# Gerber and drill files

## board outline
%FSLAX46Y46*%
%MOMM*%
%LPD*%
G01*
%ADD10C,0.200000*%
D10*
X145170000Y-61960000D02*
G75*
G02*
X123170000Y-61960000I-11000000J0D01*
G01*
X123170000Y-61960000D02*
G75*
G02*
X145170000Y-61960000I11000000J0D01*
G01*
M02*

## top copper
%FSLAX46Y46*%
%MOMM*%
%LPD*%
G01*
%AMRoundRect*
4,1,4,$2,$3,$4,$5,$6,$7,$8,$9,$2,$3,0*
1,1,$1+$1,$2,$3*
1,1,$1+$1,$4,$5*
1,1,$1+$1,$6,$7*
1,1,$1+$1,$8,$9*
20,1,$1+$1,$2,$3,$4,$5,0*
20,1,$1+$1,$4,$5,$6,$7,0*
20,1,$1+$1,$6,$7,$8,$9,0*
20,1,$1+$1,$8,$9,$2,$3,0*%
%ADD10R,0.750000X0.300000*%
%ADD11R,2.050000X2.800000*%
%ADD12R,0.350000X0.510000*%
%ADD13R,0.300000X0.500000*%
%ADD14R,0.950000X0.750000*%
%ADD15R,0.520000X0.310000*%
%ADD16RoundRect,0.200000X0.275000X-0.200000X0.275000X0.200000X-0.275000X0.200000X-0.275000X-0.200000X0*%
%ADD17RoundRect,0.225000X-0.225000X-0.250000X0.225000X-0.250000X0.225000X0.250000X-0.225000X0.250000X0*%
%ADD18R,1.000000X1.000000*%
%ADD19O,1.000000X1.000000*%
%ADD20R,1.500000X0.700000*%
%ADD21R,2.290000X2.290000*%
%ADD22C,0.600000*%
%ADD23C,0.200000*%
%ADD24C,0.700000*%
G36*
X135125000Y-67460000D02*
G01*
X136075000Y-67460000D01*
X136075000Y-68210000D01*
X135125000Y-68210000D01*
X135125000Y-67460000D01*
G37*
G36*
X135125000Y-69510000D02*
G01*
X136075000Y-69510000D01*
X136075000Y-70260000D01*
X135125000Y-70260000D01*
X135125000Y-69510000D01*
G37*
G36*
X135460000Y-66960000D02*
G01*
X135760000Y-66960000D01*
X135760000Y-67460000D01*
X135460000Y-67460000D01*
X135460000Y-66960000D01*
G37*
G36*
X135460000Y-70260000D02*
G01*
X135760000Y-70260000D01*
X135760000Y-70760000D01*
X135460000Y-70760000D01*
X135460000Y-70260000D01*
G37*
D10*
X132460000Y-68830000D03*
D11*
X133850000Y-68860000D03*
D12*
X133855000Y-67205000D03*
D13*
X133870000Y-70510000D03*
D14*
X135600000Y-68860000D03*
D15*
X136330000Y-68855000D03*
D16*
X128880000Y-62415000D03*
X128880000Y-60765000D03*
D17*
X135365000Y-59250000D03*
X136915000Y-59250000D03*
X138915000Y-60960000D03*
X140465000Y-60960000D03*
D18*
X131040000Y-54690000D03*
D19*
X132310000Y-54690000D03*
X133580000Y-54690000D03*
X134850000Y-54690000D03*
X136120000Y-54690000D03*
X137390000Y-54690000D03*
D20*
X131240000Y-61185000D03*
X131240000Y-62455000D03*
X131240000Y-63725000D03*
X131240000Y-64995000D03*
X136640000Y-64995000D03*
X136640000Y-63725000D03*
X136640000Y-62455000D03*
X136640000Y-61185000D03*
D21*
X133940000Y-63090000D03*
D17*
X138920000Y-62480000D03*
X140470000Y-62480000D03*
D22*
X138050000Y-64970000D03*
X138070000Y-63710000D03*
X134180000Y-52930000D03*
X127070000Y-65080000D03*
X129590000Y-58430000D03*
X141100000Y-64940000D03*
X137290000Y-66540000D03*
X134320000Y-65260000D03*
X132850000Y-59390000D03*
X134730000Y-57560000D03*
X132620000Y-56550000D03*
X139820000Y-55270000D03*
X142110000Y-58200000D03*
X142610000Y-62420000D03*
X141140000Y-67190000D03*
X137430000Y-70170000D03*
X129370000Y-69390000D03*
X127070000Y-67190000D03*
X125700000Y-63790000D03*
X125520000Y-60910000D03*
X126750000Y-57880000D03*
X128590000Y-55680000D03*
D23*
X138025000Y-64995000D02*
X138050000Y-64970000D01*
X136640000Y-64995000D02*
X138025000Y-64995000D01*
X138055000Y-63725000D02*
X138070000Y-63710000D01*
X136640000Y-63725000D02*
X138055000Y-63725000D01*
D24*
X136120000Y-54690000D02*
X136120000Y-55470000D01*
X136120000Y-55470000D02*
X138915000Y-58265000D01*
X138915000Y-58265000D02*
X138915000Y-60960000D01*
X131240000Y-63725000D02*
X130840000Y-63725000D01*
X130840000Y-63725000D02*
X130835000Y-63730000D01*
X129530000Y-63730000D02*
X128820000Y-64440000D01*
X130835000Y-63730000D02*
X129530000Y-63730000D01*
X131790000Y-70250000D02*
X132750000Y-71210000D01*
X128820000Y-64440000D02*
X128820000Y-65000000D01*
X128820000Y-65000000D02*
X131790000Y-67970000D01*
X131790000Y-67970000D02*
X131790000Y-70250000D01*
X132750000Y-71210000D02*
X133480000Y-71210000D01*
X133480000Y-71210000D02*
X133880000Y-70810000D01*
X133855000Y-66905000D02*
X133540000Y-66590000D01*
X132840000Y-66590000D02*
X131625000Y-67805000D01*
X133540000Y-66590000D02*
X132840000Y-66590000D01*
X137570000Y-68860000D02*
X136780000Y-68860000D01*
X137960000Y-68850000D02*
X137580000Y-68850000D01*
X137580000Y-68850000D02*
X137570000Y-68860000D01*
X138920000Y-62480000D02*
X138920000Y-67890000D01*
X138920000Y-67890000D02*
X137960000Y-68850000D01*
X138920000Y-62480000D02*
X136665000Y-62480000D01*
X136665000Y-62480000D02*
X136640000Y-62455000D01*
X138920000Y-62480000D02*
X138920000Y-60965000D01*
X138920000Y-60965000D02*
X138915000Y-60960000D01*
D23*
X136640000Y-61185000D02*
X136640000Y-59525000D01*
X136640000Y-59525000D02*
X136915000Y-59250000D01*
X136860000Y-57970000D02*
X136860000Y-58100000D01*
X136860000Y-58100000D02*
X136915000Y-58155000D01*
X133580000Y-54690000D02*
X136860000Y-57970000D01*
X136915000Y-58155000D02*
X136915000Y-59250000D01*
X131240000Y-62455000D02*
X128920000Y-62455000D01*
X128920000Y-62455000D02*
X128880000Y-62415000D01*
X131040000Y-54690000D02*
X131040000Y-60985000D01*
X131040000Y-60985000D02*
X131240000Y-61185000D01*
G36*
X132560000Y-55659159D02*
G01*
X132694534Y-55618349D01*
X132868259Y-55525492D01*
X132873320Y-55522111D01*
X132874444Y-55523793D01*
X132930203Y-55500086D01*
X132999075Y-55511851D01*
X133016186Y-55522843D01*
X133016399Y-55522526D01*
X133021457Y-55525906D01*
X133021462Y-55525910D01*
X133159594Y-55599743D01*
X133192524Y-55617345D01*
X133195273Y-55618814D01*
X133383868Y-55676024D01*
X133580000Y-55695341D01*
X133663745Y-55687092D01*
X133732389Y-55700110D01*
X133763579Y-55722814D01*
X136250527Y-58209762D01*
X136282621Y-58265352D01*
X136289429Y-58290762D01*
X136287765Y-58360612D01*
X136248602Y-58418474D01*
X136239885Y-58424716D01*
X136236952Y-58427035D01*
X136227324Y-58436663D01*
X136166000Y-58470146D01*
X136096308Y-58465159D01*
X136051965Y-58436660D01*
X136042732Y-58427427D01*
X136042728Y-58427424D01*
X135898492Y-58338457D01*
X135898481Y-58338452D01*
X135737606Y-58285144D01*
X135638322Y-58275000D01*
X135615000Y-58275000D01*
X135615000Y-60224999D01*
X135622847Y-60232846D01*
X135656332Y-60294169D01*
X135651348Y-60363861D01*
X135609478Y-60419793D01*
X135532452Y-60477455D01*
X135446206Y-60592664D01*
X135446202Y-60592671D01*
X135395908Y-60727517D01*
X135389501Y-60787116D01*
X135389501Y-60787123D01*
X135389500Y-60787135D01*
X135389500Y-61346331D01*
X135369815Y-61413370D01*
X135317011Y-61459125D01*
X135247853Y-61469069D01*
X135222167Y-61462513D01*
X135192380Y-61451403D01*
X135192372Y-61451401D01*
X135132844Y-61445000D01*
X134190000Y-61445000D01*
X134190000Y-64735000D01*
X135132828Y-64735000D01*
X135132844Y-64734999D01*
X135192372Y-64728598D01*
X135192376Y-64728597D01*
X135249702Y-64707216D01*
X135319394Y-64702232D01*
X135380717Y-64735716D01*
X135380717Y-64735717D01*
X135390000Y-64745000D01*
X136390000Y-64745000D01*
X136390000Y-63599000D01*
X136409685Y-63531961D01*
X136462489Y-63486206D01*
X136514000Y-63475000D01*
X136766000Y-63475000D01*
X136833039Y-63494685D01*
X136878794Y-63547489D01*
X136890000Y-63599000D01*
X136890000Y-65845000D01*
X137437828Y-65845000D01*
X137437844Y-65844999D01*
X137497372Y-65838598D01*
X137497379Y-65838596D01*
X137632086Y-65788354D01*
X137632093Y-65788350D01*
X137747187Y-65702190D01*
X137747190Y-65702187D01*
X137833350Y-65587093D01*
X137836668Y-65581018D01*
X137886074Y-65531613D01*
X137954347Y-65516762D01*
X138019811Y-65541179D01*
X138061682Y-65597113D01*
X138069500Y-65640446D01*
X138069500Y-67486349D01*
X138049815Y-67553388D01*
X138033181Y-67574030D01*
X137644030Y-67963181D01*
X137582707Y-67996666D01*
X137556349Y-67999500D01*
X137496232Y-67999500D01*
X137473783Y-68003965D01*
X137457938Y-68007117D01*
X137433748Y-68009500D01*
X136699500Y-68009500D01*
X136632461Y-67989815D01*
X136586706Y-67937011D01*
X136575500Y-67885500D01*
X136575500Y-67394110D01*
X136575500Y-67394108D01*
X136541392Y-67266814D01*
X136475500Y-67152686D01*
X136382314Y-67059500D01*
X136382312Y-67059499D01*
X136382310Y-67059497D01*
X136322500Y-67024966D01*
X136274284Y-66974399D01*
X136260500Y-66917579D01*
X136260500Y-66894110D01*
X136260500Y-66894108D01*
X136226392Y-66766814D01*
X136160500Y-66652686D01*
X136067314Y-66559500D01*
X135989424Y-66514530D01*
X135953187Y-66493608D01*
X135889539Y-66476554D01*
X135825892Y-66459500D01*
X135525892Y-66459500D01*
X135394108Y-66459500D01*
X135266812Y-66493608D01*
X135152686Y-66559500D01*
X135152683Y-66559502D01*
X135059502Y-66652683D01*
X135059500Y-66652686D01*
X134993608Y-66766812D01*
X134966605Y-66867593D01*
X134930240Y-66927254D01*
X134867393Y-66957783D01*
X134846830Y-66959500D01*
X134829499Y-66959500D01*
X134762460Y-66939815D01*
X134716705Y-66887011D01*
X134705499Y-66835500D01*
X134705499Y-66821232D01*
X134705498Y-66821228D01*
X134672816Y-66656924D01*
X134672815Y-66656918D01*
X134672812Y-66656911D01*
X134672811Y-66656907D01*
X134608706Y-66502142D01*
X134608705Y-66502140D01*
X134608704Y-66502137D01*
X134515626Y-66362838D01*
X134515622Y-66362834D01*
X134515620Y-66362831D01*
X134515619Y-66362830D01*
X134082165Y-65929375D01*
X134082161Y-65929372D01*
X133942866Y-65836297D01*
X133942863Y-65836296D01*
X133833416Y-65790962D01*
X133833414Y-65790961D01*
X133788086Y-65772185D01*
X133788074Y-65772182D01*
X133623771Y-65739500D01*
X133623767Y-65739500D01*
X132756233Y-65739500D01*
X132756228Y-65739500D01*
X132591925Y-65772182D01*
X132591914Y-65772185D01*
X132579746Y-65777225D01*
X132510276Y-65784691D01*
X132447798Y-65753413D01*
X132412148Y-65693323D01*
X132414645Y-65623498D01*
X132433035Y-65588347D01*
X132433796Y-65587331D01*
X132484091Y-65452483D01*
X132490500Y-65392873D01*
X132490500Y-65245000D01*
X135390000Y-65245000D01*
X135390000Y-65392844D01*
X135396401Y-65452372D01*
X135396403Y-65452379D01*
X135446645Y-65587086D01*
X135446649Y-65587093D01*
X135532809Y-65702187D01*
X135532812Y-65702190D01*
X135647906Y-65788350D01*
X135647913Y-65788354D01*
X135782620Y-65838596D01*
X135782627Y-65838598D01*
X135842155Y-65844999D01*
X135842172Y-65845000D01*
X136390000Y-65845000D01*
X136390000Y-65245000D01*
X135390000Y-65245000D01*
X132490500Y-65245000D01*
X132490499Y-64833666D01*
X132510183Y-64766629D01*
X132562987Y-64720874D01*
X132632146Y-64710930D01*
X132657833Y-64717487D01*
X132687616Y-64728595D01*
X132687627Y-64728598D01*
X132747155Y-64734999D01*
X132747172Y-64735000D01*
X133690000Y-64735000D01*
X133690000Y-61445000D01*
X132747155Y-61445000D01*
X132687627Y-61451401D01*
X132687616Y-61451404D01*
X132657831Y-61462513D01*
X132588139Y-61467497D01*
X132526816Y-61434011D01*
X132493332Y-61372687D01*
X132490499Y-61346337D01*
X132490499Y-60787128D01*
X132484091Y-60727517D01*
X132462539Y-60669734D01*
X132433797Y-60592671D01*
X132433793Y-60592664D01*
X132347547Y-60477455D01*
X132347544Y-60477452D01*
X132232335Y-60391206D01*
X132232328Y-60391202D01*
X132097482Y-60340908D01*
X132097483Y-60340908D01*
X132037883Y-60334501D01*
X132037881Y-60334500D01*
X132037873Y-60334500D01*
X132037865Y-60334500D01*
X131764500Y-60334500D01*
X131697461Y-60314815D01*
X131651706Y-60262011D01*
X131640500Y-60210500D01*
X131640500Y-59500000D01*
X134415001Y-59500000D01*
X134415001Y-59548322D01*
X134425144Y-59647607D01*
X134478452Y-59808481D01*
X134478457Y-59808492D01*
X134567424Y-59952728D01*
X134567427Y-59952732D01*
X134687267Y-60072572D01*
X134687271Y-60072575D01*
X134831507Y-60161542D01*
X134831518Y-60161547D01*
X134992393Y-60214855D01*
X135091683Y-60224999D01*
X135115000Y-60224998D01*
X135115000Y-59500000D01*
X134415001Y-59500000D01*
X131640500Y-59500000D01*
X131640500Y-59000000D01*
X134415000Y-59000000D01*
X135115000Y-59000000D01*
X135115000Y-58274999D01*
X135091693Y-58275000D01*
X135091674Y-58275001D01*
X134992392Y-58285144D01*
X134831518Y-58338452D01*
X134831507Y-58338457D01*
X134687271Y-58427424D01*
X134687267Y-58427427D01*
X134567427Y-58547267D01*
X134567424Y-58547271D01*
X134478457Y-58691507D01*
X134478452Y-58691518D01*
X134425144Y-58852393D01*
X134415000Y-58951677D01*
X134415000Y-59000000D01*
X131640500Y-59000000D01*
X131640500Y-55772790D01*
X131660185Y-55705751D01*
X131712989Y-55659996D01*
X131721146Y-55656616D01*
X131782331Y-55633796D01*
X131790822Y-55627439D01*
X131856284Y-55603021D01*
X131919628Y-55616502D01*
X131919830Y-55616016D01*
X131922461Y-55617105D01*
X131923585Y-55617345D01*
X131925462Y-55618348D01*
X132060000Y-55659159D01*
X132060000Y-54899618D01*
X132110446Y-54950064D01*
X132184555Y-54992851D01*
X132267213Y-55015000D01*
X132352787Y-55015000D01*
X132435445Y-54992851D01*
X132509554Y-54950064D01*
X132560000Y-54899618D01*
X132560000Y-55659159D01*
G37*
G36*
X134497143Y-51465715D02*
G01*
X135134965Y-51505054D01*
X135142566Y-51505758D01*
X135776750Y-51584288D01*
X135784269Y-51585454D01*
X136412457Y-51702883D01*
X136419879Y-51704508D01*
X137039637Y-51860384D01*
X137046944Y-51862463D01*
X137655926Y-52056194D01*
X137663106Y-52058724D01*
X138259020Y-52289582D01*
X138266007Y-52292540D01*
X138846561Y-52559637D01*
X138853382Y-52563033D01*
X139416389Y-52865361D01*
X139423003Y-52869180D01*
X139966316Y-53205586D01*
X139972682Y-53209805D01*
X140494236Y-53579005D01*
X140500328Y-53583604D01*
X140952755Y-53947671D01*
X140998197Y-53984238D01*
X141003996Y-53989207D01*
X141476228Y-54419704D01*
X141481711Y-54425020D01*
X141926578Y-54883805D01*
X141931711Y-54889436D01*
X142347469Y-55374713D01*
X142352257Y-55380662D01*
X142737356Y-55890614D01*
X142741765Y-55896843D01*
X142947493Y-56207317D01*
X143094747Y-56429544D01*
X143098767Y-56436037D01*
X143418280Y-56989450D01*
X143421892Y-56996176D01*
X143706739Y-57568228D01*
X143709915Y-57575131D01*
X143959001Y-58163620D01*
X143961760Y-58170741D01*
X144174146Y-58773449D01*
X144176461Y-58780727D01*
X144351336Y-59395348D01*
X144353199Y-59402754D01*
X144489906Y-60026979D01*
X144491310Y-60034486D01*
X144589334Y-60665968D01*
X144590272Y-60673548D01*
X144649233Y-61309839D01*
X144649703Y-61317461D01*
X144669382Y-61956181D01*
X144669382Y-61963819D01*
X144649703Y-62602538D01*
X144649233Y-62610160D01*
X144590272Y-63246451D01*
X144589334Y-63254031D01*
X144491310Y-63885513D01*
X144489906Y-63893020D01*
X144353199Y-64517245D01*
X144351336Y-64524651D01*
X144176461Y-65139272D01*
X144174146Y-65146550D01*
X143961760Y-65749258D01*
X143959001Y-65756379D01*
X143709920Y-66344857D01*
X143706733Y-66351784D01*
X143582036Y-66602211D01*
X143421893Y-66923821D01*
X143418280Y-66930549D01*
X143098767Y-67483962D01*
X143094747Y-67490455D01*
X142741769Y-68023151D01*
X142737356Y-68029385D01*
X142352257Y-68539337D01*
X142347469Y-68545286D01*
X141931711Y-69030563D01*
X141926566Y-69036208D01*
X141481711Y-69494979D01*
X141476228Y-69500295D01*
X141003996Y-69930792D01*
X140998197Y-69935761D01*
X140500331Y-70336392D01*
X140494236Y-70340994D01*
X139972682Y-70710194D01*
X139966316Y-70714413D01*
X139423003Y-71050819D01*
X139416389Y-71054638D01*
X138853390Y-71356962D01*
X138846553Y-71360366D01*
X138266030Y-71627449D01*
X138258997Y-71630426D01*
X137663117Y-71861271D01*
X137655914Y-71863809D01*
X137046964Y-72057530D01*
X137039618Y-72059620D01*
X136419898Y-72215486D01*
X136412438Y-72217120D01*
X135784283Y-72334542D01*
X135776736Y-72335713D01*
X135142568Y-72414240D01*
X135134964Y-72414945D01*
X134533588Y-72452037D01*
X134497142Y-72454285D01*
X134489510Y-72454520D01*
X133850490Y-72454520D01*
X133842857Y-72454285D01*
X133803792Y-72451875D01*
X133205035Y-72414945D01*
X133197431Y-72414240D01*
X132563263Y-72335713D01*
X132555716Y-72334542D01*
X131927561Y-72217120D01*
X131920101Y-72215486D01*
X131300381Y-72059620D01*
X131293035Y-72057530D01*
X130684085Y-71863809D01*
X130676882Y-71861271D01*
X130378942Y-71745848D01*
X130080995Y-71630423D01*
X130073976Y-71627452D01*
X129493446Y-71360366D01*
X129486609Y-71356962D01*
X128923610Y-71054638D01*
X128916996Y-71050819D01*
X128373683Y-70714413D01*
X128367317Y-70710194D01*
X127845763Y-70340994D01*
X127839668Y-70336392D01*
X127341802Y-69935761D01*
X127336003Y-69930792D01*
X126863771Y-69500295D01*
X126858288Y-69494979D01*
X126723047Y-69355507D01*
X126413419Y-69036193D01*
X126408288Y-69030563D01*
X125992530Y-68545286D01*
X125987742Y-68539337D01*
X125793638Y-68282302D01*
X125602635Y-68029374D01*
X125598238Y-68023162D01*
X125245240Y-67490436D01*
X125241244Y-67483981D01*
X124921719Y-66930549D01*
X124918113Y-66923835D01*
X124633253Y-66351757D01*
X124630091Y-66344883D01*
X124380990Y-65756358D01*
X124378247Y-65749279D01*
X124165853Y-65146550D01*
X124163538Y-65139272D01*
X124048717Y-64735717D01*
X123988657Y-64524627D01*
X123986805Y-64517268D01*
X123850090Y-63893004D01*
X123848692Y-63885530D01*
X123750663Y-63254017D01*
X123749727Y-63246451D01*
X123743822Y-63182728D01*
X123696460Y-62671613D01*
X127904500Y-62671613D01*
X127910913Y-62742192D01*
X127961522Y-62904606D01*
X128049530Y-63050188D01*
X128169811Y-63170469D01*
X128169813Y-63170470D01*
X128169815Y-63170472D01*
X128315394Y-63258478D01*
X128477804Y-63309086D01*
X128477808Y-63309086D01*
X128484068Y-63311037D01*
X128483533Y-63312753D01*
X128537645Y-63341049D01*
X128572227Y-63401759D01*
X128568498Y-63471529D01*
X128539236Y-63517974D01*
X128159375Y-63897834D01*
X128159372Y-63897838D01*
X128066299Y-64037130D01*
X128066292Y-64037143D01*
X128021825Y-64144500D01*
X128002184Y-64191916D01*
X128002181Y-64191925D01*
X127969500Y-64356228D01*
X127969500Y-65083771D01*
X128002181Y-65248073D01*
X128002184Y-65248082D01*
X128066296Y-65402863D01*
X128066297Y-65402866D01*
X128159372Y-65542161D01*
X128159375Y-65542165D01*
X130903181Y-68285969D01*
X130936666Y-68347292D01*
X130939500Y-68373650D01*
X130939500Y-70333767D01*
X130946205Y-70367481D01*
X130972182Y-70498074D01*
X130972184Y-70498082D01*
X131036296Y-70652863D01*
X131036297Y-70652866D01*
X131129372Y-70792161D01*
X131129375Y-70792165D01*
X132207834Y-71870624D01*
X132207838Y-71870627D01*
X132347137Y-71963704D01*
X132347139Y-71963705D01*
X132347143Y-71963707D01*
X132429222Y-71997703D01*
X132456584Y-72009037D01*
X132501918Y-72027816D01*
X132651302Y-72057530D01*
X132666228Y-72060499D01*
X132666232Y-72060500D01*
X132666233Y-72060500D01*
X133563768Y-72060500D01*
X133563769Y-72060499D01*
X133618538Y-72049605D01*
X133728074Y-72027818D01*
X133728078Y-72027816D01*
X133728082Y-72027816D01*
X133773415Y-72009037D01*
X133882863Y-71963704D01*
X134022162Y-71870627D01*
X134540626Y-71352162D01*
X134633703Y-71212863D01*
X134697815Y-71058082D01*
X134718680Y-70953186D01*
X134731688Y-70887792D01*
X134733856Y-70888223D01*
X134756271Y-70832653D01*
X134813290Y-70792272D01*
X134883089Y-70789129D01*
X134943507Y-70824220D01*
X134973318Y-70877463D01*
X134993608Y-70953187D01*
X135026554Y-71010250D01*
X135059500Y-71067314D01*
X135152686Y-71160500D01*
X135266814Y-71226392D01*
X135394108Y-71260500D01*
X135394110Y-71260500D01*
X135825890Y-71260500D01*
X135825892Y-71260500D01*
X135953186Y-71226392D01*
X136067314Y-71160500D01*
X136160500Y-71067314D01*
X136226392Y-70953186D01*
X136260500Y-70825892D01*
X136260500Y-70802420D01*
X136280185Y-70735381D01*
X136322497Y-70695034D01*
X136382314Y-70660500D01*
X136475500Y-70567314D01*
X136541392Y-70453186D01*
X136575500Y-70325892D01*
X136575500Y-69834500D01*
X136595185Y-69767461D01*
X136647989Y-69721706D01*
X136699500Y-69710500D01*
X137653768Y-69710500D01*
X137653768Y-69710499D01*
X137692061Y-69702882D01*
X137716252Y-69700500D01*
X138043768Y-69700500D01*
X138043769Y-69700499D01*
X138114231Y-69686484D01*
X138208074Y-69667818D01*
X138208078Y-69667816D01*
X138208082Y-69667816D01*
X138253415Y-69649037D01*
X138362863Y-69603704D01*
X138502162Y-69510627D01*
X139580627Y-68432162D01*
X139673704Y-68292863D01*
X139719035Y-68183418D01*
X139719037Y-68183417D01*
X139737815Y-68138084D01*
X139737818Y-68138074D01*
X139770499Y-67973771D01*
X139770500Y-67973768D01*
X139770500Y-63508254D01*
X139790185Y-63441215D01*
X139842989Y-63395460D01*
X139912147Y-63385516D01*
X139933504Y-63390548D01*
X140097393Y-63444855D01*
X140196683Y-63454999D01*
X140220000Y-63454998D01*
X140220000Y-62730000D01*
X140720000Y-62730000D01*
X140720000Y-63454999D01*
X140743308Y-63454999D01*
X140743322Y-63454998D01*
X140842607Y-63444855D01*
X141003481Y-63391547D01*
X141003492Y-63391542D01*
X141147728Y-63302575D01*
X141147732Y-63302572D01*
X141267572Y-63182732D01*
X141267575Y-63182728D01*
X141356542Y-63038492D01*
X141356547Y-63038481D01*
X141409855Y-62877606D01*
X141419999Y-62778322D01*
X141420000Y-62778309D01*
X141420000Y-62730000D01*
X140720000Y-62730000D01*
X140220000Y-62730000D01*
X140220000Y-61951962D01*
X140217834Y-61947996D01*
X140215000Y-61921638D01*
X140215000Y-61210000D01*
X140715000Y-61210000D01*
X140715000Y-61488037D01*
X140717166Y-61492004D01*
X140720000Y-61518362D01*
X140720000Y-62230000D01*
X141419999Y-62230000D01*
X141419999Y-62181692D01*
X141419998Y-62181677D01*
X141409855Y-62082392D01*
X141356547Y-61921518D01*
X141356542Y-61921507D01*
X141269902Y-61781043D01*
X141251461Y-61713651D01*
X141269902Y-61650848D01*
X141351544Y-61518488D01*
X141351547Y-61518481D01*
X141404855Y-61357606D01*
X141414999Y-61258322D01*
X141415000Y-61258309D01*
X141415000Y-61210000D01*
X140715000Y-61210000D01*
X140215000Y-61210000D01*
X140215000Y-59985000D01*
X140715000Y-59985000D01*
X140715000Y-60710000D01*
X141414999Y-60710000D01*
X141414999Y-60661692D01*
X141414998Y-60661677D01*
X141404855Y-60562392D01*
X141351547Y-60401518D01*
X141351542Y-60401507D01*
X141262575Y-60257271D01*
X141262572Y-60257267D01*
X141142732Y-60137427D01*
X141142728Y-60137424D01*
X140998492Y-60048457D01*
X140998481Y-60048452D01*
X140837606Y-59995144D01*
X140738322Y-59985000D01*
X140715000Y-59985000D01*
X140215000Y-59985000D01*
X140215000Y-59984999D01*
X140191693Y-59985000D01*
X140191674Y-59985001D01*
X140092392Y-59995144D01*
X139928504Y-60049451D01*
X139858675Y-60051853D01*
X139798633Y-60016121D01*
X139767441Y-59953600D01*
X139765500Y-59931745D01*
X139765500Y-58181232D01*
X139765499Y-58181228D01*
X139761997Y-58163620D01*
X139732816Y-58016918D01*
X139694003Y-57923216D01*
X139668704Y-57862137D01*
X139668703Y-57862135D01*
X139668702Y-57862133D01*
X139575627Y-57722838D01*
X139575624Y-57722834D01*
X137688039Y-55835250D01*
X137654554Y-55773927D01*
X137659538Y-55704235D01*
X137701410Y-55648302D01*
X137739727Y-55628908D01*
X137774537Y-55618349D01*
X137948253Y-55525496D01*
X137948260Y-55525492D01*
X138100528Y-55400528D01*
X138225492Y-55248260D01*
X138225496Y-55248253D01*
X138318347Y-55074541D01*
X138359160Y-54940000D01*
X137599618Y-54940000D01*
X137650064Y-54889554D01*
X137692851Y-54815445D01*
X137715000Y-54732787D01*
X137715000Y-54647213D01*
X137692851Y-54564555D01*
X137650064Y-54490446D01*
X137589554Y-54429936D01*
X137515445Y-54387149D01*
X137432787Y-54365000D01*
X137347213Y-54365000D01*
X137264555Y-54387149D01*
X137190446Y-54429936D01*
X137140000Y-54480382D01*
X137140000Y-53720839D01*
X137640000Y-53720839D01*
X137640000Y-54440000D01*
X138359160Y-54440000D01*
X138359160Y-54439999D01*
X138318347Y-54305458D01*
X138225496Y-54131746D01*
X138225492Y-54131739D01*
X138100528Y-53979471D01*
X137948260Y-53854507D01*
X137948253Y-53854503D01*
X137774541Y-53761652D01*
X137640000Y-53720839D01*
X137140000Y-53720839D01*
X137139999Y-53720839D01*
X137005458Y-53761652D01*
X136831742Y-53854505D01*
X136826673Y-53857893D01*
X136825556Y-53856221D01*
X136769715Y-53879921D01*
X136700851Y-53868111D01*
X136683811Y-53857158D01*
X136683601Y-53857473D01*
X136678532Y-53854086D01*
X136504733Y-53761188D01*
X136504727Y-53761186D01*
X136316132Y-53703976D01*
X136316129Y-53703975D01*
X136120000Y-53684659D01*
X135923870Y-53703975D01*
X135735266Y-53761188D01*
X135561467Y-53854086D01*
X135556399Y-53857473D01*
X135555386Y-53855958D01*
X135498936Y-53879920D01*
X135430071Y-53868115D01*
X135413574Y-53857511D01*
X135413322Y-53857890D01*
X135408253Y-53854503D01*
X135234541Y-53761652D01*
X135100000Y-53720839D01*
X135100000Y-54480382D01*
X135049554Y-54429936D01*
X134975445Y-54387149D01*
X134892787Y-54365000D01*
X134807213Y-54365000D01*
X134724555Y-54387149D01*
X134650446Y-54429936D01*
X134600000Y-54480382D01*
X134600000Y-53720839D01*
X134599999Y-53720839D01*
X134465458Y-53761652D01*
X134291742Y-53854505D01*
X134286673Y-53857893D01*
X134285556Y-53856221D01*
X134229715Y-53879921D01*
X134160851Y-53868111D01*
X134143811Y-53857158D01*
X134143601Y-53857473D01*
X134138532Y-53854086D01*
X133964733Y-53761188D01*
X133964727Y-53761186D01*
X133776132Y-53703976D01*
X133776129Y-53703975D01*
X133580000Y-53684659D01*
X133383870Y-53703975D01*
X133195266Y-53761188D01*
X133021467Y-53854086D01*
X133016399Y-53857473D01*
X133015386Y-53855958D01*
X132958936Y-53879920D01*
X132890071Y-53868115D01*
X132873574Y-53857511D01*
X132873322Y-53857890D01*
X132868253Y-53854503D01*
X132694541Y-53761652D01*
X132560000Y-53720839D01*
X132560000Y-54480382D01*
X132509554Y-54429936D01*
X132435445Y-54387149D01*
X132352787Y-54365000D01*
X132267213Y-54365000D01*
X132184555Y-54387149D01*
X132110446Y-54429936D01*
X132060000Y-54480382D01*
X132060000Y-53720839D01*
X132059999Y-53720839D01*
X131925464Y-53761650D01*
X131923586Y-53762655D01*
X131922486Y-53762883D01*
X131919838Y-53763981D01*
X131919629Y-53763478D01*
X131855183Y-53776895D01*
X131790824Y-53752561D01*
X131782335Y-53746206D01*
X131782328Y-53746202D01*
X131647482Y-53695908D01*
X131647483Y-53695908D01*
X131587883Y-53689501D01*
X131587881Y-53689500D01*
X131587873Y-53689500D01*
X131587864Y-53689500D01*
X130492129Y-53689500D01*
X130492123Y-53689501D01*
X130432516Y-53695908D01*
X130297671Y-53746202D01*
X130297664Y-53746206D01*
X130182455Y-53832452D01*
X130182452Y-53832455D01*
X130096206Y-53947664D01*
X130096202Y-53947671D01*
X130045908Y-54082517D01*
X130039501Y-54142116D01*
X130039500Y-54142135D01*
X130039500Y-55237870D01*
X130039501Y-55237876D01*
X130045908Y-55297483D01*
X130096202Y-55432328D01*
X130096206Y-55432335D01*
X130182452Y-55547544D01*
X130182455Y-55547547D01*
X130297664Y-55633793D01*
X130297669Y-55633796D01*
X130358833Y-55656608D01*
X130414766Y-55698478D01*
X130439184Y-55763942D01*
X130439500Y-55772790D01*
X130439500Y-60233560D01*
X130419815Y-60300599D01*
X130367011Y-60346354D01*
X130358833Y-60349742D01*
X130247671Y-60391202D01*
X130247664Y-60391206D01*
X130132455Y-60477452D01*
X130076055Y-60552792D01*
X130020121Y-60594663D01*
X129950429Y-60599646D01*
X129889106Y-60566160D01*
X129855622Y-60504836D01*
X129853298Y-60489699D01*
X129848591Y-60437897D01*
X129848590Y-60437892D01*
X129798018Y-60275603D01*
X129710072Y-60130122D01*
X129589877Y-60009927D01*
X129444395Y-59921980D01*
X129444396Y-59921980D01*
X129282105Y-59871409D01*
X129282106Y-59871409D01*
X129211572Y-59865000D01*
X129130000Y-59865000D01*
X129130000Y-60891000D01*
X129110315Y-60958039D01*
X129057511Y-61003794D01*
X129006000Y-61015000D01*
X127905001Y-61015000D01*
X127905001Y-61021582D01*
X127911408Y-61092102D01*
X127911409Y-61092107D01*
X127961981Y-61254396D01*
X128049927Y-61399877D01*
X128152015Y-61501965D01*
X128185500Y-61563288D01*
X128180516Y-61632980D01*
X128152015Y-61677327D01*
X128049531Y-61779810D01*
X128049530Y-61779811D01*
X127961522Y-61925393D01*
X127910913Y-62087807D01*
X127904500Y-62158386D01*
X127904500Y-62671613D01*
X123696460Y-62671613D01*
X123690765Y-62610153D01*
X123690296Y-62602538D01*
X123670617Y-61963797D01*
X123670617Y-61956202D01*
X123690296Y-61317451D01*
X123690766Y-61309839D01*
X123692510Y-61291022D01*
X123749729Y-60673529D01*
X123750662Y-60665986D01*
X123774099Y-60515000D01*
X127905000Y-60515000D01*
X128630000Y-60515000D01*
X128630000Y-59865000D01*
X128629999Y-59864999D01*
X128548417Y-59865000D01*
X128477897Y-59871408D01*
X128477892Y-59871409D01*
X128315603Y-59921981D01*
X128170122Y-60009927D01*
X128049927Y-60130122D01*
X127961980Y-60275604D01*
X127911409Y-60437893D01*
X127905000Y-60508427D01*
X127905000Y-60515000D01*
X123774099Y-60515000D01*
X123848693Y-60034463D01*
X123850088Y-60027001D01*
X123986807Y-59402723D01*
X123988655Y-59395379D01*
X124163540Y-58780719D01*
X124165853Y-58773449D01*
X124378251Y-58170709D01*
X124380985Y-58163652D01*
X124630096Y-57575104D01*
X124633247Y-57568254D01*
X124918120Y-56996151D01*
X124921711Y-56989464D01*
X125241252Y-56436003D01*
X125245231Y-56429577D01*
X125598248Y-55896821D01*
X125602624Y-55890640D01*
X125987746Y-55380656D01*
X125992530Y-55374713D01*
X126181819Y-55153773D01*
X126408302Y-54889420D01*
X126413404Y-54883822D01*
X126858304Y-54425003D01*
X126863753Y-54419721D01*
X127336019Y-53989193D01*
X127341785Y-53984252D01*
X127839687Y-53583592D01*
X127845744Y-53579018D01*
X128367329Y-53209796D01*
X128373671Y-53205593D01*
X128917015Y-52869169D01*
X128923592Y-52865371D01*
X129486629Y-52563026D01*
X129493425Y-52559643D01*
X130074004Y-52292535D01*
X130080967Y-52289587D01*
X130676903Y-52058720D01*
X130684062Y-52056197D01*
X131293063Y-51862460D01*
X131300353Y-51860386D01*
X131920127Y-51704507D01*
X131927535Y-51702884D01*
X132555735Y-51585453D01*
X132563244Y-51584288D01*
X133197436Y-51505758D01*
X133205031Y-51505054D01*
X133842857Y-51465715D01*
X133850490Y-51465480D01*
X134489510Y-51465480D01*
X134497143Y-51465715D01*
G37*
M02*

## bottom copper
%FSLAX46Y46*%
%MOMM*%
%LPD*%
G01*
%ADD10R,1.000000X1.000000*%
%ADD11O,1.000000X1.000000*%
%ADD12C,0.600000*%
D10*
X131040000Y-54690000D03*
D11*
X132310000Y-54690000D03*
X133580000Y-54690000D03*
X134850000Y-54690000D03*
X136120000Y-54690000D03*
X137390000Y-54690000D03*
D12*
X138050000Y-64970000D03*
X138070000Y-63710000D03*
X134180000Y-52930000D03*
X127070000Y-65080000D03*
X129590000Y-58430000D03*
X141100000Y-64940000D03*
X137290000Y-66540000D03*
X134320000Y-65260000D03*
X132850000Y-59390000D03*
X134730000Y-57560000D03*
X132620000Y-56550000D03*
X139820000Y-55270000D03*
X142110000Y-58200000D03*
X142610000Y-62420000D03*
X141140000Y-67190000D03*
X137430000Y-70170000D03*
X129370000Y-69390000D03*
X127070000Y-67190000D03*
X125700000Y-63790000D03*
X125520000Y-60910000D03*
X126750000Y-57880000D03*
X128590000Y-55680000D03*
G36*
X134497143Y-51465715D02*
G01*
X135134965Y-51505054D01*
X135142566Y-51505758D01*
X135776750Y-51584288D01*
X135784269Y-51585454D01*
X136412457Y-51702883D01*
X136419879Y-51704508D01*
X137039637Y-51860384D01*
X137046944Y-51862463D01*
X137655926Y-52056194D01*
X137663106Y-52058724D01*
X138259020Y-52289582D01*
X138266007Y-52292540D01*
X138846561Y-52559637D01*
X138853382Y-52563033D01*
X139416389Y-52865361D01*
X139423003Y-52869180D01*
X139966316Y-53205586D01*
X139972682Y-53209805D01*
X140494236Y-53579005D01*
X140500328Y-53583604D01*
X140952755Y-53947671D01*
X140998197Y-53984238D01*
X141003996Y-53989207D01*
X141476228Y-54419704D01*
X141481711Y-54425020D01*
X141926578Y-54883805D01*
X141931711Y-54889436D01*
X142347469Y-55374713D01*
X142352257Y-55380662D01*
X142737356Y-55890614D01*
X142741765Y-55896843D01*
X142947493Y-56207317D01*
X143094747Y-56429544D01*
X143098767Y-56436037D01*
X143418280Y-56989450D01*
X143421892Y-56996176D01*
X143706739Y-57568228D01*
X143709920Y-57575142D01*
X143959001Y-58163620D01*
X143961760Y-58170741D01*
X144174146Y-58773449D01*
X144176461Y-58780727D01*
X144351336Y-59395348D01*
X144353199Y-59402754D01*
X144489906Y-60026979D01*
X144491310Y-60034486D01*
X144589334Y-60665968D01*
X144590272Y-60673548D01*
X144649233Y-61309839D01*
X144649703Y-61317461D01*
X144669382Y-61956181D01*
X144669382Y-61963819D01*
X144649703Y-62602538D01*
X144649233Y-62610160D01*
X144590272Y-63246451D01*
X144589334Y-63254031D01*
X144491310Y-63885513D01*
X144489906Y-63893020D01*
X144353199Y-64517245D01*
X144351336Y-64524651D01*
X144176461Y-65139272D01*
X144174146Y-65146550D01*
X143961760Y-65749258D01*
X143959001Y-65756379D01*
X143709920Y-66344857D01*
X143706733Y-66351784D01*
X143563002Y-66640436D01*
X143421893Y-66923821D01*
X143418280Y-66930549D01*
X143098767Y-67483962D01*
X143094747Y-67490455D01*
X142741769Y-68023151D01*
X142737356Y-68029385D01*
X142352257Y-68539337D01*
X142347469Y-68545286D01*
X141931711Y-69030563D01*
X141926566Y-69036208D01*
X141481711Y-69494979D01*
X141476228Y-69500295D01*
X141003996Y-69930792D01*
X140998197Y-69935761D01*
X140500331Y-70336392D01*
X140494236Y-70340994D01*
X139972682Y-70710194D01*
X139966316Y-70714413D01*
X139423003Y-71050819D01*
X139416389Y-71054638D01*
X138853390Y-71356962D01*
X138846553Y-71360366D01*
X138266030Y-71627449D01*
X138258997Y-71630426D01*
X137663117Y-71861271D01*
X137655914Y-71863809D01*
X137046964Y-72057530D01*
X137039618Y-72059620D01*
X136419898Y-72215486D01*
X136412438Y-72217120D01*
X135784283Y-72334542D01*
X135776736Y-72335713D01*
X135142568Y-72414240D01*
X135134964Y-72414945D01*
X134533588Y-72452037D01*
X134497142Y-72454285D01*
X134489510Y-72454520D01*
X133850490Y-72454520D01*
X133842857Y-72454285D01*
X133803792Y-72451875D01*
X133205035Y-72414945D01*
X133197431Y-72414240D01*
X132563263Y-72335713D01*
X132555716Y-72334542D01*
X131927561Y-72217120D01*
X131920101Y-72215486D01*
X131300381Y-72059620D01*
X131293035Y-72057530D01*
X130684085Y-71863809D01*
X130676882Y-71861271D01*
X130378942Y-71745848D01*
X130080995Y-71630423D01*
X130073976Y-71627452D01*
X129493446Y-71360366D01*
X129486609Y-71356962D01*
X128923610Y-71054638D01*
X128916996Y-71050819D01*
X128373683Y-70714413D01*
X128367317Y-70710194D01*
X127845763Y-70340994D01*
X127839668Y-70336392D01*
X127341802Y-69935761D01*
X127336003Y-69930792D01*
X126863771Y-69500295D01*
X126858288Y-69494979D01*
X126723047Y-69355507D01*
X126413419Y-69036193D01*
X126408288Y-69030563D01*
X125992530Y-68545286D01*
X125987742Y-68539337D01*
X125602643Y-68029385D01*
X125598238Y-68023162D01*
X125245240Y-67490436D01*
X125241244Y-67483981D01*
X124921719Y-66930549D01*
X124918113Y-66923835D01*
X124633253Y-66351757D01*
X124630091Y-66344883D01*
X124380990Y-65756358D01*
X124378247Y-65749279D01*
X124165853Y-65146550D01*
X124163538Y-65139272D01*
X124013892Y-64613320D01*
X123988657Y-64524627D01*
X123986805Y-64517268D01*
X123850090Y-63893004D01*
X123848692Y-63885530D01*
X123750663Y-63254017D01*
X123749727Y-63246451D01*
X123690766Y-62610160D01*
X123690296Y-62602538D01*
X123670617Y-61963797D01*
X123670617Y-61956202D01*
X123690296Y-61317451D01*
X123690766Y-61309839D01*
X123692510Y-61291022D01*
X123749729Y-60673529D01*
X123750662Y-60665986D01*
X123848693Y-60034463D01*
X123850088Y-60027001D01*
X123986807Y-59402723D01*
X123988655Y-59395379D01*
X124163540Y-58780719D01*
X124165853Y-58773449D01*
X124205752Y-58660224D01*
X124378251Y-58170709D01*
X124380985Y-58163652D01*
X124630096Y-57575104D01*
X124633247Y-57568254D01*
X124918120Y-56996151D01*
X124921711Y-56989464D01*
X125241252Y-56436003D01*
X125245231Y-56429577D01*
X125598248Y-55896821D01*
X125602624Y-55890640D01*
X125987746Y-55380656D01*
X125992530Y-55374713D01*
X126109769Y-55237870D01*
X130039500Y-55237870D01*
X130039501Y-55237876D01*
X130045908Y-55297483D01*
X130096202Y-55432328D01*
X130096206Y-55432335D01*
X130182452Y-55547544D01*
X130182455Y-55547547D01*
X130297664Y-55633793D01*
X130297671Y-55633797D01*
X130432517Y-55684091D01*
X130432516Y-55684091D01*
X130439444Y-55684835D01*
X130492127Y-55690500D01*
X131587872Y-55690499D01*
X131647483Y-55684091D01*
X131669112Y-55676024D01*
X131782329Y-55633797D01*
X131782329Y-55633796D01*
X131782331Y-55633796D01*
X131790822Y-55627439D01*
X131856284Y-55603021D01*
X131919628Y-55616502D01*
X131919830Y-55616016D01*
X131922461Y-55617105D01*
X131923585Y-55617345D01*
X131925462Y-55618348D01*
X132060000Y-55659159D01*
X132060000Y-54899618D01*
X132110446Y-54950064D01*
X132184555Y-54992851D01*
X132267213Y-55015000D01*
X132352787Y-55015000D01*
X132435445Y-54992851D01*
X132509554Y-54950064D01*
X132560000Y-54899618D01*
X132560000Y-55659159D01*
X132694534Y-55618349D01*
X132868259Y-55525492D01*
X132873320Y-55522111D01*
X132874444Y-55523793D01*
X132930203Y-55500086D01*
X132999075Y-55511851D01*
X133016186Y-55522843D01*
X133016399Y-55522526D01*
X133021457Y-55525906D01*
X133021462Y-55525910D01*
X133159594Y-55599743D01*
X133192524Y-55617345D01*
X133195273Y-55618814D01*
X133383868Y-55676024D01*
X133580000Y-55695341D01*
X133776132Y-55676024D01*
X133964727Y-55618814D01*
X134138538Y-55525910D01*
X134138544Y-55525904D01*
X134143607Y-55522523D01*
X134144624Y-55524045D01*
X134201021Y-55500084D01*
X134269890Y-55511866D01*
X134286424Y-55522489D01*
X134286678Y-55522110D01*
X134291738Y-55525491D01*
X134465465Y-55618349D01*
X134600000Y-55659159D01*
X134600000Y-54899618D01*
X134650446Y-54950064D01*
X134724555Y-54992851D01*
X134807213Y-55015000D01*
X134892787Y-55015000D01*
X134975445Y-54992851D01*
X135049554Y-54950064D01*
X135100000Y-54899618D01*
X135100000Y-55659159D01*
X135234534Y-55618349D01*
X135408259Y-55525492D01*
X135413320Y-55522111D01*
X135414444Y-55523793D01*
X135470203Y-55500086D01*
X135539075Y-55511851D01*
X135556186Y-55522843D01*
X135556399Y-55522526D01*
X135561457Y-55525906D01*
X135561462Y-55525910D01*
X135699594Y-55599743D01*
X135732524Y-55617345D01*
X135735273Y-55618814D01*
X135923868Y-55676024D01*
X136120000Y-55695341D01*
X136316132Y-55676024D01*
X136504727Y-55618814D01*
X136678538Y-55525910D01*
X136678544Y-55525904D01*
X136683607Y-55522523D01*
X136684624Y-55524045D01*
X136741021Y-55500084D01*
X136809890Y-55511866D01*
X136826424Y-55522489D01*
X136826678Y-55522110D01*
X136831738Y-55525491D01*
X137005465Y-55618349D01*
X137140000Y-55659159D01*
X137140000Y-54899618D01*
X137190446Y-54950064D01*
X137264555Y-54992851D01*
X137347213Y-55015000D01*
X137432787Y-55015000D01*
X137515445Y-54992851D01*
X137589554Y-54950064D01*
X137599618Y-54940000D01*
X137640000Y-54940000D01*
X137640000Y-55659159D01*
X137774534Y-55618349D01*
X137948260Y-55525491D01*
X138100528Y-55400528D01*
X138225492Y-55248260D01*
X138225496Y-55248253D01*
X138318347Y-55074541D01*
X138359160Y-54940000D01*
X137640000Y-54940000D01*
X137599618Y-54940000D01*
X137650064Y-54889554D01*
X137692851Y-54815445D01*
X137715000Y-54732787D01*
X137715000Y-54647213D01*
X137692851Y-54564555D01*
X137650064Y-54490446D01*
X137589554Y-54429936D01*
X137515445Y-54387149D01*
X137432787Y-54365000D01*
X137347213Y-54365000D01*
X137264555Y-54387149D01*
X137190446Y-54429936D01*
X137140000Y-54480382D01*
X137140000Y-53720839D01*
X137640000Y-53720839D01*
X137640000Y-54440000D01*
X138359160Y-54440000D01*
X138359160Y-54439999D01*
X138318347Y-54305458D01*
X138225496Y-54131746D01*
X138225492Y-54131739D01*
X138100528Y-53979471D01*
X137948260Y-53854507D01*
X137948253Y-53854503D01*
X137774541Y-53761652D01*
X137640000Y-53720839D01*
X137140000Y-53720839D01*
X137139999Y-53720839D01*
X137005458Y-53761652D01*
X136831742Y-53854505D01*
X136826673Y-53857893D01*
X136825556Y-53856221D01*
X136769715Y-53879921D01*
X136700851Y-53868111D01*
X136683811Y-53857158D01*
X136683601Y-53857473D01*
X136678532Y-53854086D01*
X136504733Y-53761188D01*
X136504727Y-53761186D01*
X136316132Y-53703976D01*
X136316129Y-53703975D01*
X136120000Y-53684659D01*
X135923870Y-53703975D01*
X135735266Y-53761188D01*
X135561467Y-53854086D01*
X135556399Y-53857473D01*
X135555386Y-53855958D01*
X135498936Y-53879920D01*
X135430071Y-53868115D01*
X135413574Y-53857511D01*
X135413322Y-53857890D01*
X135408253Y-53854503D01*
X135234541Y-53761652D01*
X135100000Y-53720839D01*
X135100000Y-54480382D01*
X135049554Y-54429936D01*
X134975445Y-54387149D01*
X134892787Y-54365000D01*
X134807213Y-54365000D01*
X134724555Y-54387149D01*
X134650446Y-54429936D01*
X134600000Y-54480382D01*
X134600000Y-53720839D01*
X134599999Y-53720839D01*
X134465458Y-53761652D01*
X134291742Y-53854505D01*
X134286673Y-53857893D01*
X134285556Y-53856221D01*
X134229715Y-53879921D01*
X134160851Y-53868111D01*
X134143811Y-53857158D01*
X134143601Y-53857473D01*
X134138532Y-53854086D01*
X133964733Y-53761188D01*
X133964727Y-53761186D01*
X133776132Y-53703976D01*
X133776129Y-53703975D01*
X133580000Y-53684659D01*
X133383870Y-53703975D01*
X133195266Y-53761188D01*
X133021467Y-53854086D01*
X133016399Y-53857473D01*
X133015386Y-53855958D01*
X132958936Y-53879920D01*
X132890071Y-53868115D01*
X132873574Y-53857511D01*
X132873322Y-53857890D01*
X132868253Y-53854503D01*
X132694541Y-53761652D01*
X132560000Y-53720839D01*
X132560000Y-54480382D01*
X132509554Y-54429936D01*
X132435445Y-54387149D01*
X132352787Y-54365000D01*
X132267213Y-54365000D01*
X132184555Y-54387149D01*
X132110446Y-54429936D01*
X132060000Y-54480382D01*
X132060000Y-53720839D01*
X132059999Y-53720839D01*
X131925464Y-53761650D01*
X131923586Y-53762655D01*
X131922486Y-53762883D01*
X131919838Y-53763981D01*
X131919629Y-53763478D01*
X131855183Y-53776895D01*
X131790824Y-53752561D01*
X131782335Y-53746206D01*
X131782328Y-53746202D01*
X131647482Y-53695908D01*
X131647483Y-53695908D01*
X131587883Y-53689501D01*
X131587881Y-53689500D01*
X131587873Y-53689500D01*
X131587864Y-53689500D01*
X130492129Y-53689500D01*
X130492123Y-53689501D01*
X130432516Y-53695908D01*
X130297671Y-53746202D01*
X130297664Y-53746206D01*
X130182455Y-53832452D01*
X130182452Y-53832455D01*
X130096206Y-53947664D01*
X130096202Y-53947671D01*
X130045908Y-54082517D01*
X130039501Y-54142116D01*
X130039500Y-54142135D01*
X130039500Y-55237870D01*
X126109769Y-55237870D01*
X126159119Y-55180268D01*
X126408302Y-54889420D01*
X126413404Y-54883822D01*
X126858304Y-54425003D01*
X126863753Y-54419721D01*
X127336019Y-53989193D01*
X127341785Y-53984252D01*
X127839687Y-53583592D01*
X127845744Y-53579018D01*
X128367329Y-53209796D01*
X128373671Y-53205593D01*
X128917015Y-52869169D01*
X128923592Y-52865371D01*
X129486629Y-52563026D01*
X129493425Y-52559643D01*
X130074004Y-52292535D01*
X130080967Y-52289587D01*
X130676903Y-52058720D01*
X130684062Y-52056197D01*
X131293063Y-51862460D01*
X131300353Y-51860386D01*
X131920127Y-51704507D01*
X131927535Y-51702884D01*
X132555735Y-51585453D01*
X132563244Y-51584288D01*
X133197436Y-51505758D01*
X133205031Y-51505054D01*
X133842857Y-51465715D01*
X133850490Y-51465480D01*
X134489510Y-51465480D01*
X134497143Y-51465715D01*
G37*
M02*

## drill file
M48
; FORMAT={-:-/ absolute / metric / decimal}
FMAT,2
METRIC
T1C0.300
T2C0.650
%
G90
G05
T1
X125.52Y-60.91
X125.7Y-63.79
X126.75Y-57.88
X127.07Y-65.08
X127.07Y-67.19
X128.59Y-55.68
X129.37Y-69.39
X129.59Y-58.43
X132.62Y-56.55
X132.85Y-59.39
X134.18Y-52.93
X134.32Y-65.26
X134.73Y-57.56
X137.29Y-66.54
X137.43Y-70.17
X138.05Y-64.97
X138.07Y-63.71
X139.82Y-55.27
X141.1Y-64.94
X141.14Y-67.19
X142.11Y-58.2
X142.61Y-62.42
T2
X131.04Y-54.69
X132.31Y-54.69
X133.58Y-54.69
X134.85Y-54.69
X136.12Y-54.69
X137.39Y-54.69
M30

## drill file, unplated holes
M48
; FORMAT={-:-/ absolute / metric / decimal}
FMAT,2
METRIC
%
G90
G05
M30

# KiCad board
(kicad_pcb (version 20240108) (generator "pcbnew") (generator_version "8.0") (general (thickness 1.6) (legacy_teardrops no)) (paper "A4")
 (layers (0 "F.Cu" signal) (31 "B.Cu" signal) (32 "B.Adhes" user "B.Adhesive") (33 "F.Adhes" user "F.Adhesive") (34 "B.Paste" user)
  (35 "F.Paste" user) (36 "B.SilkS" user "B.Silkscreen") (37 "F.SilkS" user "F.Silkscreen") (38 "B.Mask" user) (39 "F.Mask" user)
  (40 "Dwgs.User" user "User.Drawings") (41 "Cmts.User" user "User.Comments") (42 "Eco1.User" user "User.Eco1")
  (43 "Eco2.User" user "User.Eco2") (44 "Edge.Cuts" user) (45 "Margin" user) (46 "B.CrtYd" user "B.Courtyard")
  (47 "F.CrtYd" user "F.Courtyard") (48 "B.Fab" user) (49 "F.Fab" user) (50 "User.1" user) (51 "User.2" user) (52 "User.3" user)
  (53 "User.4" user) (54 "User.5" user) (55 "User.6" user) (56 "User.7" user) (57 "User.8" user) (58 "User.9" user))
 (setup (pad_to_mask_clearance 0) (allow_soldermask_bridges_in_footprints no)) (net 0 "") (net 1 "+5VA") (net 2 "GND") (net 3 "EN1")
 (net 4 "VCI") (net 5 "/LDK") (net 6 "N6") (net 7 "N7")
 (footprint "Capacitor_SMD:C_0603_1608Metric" (layer "F.Cu") (at 139.695 62.48)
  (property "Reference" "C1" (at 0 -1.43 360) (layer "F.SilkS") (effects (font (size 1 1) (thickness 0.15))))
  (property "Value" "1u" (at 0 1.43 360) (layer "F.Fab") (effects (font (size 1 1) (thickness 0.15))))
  (pad "1" smd roundrect (at -0.775 0) (size 0.9 0.95) (layers "F.Cu" "F.Paste" "F.Mask") (roundrect_rratio 0.25) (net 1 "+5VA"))
  (pad "2" smd roundrect (at 0.775 0) (size 0.9 0.95) (layers "F.Cu" "F.Paste" "F.Mask") (roundrect_rratio 0.25) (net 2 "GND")))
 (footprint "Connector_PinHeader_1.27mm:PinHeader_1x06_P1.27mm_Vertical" (layer "F.Cu") (at 131.04 54.69 90)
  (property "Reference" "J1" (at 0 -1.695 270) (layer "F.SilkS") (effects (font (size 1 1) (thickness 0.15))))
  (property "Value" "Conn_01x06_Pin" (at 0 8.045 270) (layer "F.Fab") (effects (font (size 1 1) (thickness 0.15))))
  (pad "1" thru_hole rect (at 0 0 90) (size 1 1) (drill 0.65) (layers "*.Cu" "*.Mask") (remove_unused_layers no) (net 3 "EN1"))
  (pad "2" thru_hole oval (at 0 1.27 90) (size 1 1) (drill 0.65) (layers "*.Cu" "*.Mask") (remove_unused_layers no) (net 2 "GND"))
  (pad "3" thru_hole oval (at 0 2.54 90) (size 1 1) (drill 0.65) (layers "*.Cu" "*.Mask") (remove_unused_layers no) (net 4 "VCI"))
  (pad "4" thru_hole oval (at 0 3.81 90) (size 1 1) (drill 0.65) (layers "*.Cu" "*.Mask") (remove_unused_layers no) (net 2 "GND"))
  (pad "5" thru_hole oval (at 0 5.08 90) (size 1 1) (drill 0.65) (layers "*.Cu" "*.Mask") (remove_unused_layers no) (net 1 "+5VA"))
  (pad "6" thru_hole oval (at 0 6.35 90) (size 1 1) (drill 0.65) (layers "*.Cu" "*.Mask") (remove_unused_layers no) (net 2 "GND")))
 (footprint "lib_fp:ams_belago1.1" (layer "F.Cu") (at 137.12 61.92)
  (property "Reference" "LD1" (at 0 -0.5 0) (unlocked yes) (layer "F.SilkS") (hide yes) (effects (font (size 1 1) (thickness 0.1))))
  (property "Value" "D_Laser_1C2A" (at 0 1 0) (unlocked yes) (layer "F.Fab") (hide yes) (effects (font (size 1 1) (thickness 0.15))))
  (fp_rect (start -1.995 5.54) (end -1.045 6.29) (stroke (width 0) (type solid)) (fill solid) (layer "F.Cu"))
  (fp_rect (start -1.995 7.59) (end -1.045 8.34) (stroke (width 0) (type solid)) (fill solid) (layer "F.Cu"))
  (fp_rect (start -1.66 5.04) (end -1.36 5.54) (stroke (width 0) (type solid)) (fill solid) (layer "F.Cu"))
  (fp_rect (start -1.66 8.34) (end -1.36 8.84) (stroke (width 0) (type solid)) (fill solid) (layer "F.Cu"))
  (pad "1" smd rect (at -4.66 6.91) (size 0.75 0.3) (layers "F.Cu" "F.Paste" "F.Mask") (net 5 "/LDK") (thermal_bridge_angle 45))
  (pad "1" smd rect (at -3.27 6.94) (size 2.05 2.8) (layers "F.Cu" "F.Paste" "F.Mask") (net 5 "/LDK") (thermal_bridge_angle 45))
  (pad "1" smd rect (at -3.265 5.285) (size 0.35 0.51) (layers "F.Cu" "F.Paste" "F.Mask") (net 5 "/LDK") (thermal_bridge_angle 45))
  (pad "1" smd rect (at -3.25 8.59) (size 0.3 0.5) (layers "F.Cu" "F.Paste" "F.Mask") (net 5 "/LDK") (thermal_bridge_angle 45))
  (pad "2" smd rect (at -1.52 6.94) (size 0.95 0.75) (layers "F.Cu" "F.Paste" "F.Mask") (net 1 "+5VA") (thermal_bridge_angle 45))
  (pad "2" smd rect (at -0.79 6.935) (size 0.52 0.31) (layers "F.Cu" "F.Paste" "F.Mask") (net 1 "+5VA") (thermal_bridge_angle 45)))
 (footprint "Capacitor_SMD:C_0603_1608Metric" (layer "F.Cu") (at 136.14 59.25)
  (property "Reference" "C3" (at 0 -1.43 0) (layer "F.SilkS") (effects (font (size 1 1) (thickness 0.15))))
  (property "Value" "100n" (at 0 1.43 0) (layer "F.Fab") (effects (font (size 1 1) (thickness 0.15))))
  (pad "1" smd roundrect (at -0.775 0) (size 0.9 0.95) (layers "F.Cu" "F.Paste" "F.Mask") (roundrect_rratio 0.25) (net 2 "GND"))
  (pad "2" smd roundrect (at 0.775 0) (size 0.9 0.95) (layers "F.Cu" "F.Paste" "F.Mask") (roundrect_rratio 0.25) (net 4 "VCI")))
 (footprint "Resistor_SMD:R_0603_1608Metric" (layer "F.Cu") (at 128.88 61.59 90)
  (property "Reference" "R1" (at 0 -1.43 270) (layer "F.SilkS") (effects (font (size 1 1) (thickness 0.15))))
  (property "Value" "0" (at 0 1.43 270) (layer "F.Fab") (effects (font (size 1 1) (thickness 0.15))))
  (pad "1" smd roundrect (at -0.825 0 90) (size 0.8 0.95) (layers "F.Cu" "F.Paste" "F.Mask") (roundrect_rratio 0.25) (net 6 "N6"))
  (pad "2" smd roundrect (at 0.825 0 90) (size 0.8 0.95) (layers "F.Cu" "F.Paste" "F.Mask") (roundrect_rratio 0.25) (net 2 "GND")))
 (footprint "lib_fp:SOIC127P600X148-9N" (layer "F.Cu") (at 133.94 63.09)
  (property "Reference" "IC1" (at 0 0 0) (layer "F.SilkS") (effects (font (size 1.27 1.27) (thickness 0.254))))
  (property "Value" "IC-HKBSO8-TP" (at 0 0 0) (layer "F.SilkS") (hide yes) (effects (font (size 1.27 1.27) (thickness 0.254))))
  (pad "1" smd rect (at -2.7 -1.905 90) (size 0.7 1.5) (layers "F.Cu" "F.Paste" "F.Mask") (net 3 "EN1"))
  (pad "2" smd rect (at -2.7 -0.635 90) (size 0.7 1.5) (layers "F.Cu" "F.Paste" "F.Mask") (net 6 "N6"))
  (pad "3" smd rect (at -2.7 0.635 90) (size 0.7 1.5) (layers "F.Cu" "F.Paste" "F.Mask") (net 5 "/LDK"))
  (pad "4" smd rect (at -2.7 1.905 90) (size 0.7 1.5) (layers "F.Cu" "F.Paste" "F.Mask") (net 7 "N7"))
  (pad "5" smd rect (at 2.7 1.905 90) (size 0.7 1.5) (layers "F.Cu" "F.Paste" "F.Mask") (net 2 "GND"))
  (pad "6" smd rect (at 2.7 0.635 90) (size 0.7 1.5) (layers "F.Cu" "F.Paste" "F.Mask") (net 2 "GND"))
  (pad "7" smd rect (at 2.7 -0.635 90) (size 0.7 1.5) (layers "F.Cu" "F.Paste" "F.Mask") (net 1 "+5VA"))
  (pad "8" smd rect (at 2.7 -1.905 90) (size 0.7 1.5) (layers "F.Cu" "F.Paste" "F.Mask") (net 4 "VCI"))
  (pad "9" smd rect (at 0 0) (size 2.29 2.29) (layers "F.Cu" "F.Paste" "F.Mask") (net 2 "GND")))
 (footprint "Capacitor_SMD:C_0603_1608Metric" (layer "F.Cu") (at 139.69 60.96)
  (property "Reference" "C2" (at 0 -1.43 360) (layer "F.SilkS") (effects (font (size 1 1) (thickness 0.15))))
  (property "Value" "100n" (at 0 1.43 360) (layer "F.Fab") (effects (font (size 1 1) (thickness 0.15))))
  (pad "1" smd roundrect (at -0.775 0) (size 0.9 0.95) (layers "F.Cu" "F.Paste" "F.Mask") (roundrect_rratio 0.25) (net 1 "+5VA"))
  (pad "2" smd roundrect (at 0.775 0) (size 0.9 0.95) (layers "F.Cu" "F.Paste" "F.Mask") (roundrect_rratio 0.25) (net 2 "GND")))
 (gr_circle (center 134.17 61.96) (end 145.17 61.96) (stroke (width 0.2) (type default)) (fill none) (layer "Edge.Cuts"))
 (segment (start 138.92 67.89) (end 137.96 68.85) (width 0.7) (layer "F.Cu") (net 1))
 (segment (start 136.12 55.47) (end 138.915 58.265) (width 0.7) (layer "F.Cu") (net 1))
 (segment (start 136.12 54.69) (end 136.12 55.47) (width 0.7) (layer "F.Cu") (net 1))
 (segment (start 138.92 62.48) (end 138.92 67.89) (width 0.7) (layer "F.Cu") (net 1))
 (segment (start 137.96 68.85) (end 137.58 68.85) (width 0.7) (layer "F.Cu") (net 1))
 (segment (start 136.665 62.48) (end 136.64 62.455) (width 0.7) (layer "F.Cu") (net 1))
 (segment (start 138.92 62.48) (end 136.665 62.48) (width 0.7) (layer "F.Cu") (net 1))
 (segment (start 138.92 62.48) (end 138.92 60.965) (width 0.7) (layer "F.Cu") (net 1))
 (segment (start 138.92 60.965) (end 138.915 60.96) (width 0.7) (layer "F.Cu") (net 1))
 (segment (start 137.57 68.86) (end 136.78 68.86) (width 0.7) (layer "F.Cu") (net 1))
 (segment (start 137.58 68.85) (end 137.57 68.86) (width 0.7) (layer "F.Cu") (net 1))
 (segment (start 138.915 58.265) (end 138.915 60.96) (width 0.7) (layer "F.Cu") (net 1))
 (segment (start 136.64 64.995) (end 138.025 64.995) (width 0.2) (layer "F.Cu") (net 2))
 (segment (start 138.025 64.995) (end 138.05 64.97) (width 0.2) (layer "F.Cu") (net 2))
 (segment (start 138.055 63.725) (end 138.07 63.71) (width 0.2) (layer "F.Cu") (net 2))
 (segment (start 136.64 63.725) (end 138.055 63.725) (width 0.2) (layer "F.Cu") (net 2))
 (via (at 142.61 62.42) (size 0.6) (drill 0.3) (layers "F.Cu" "B.Cu") (free yes) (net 2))
 (via (at 141.1 64.94) (size 0.6) (drill 0.3) (layers "F.Cu" "B.Cu") (free yes) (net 2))
 (via (at 138.07 63.71) (size 0.6) (drill 0.3) (layers "F.Cu" "B.Cu") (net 2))
 (via (at 127.07 65.08) (size 0.6) (drill 0.3) (layers "F.Cu" "B.Cu") (free yes) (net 2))
 (via (at 129.59 58.43) (size 0.6) (drill 0.3) (layers "F.Cu" "B.Cu") (free yes) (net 2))
 (via (at 129.37 69.39) (size 0.6) (drill 0.3) (layers "F.Cu" "B.Cu") (free yes) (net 2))
 (via (at 128.59 55.68) (size 0.6) (drill 0.3) (layers "F.Cu" "B.Cu") (free yes) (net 2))
 (via (at 134.18 52.93) (size 0.6) (drill 0.3) (layers "F.Cu" "B.Cu") (free yes) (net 2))
 (via (at 132.85 59.39) (size 0.6) (drill 0.3) (layers "F.Cu" "B.Cu") (free yes) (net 2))
 (via (at 138.05 64.97) (size 0.6) (drill 0.3) (layers "F.Cu" "B.Cu") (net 2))
 (via (at 139.82 55.27) (size 0.6) (drill 0.3) (layers "F.Cu" "B.Cu") (free yes) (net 2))
 (via (at 134.73 57.56) (size 0.6) (drill 0.3) (layers "F.Cu" "B.Cu") (free yes) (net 2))
 (via (at 137.29 66.54) (size 0.6) (drill 0.3) (layers "F.Cu" "B.Cu") (free yes) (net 2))
 (via (at 125.52 60.91) (size 0.6) (drill 0.3) (layers "F.Cu" "B.Cu") (free yes) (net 2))
 (via (at 132.62 56.55) (size 0.6) (drill 0.3) (layers "F.Cu" "B.Cu") (free yes) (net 2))
 (via (at 137.43 70.17) (size 0.6) (drill 0.3) (layers "F.Cu" "B.Cu") (free yes) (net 2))
 (via (at 141.14 67.19) (size 0.6) (drill 0.3) (layers "F.Cu" "B.Cu") (free yes) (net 2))
 (via (at 127.07 67.19) (size 0.6) (drill 0.3) (layers "F.Cu" "B.Cu") (free yes) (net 2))
 (via (at 134.32 65.26) (size 0.6) (drill 0.3) (layers "F.Cu" "B.Cu") (free yes) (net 2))
 (via (at 125.7 63.79) (size 0.6) (drill 0.3) (layers "F.Cu" "B.Cu") (free yes) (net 2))
 (via (at 142.11 58.2) (size 0.6) (drill 0.3) (layers "F.Cu" "B.Cu") (free yes) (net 2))
 (via (at 126.75 57.88) (size 0.6) (drill 0.3) (layers "F.Cu" "B.Cu") (free yes) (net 2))
 (segment (start 131.04 60.985) (end 131.24 61.185) (width 0.2) (layer "F.Cu") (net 3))
 (segment (start 131.04 54.69) (end 131.04 60.985) (width 0.2) (layer "F.Cu") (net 3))
 (segment (start 129.53 63.73) (end 128.82 64.44) (width 0.7) (layer "F.Cu") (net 5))
 (segment (start 133.54 66.59) (end 132.84 66.59) (width 0.7) (layer "F.Cu") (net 5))
 (segment (start 132.75 71.21) (end 133.48 71.21) (width 0.7) (layer "F.Cu") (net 5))
 (segment (start 133.855 66.905) (end 133.54 66.59) (width 0.7) (layer "F.Cu") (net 5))
 (segment (start 128.82 64.44) (end 128.82 65) (width 0.7) (layer "F.Cu") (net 5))
 (segment (start 131.79 67.97) (end 131.79 70.25) (width 0.7) (layer "F.Cu") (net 5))
 (segment (start 131.79 70.25) (end 132.75 71.21) (width 0.7) (layer "F.Cu") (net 5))
 (segment (start 132.84 66.59) (end 131.625 67.805) (width 0.7) (layer "F.Cu") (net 5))
 (segment (start 130.84 63.725) (end 130.835 63.73) (width 0.7) (layer "F.Cu") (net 5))
 (segment (start 133.48 71.21) (end 133.88 70.81) (width 0.7) (layer "F.Cu") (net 5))
 (segment (start 128.82 65) (end 131.79 67.97) (width 0.7) (layer "F.Cu") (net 5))
 (segment (start 131.24 63.725) (end 130.84 63.725) (width 0.7) (layer "F.Cu") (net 5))
 (segment (start 130.835 63.73) (end 129.53 63.73) (width 0.7) (layer "F.Cu") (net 5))
 (segment (start 136.915 58.155) (end 136.915 59.25) (width 0.2) (layer "F.Cu") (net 4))
 (segment (start 133.58 54.69) (end 136.86 57.97) (width 0.2) (layer "F.Cu") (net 4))
 (segment (start 136.64 59.525) (end 136.915 59.25) (width 0.2) (layer "F.Cu") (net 4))
 (segment (start 136.86 57.97) (end 136.86 58.1) (width 0.2) (layer "F.Cu") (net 4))
 (segment (start 136.86 58.1) (end 136.915 58.155) (width 0.2) (layer "F.Cu") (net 4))
 (segment (start 136.64 61.185) (end 136.64 59.525) (width 0.2) (layer "F.Cu") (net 4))
 (segment (start 131.24 62.455) (end 128.92 62.455) (width 0.2) (layer "F.Cu") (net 6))
 (segment (start 128.92 62.455) (end 128.88 62.415) (width 0.2) (layer "F.Cu") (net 6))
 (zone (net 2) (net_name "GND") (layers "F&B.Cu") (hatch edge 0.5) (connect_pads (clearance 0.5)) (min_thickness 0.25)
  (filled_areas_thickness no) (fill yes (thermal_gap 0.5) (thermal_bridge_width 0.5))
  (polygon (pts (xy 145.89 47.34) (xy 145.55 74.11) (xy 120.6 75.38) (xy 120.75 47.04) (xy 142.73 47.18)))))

